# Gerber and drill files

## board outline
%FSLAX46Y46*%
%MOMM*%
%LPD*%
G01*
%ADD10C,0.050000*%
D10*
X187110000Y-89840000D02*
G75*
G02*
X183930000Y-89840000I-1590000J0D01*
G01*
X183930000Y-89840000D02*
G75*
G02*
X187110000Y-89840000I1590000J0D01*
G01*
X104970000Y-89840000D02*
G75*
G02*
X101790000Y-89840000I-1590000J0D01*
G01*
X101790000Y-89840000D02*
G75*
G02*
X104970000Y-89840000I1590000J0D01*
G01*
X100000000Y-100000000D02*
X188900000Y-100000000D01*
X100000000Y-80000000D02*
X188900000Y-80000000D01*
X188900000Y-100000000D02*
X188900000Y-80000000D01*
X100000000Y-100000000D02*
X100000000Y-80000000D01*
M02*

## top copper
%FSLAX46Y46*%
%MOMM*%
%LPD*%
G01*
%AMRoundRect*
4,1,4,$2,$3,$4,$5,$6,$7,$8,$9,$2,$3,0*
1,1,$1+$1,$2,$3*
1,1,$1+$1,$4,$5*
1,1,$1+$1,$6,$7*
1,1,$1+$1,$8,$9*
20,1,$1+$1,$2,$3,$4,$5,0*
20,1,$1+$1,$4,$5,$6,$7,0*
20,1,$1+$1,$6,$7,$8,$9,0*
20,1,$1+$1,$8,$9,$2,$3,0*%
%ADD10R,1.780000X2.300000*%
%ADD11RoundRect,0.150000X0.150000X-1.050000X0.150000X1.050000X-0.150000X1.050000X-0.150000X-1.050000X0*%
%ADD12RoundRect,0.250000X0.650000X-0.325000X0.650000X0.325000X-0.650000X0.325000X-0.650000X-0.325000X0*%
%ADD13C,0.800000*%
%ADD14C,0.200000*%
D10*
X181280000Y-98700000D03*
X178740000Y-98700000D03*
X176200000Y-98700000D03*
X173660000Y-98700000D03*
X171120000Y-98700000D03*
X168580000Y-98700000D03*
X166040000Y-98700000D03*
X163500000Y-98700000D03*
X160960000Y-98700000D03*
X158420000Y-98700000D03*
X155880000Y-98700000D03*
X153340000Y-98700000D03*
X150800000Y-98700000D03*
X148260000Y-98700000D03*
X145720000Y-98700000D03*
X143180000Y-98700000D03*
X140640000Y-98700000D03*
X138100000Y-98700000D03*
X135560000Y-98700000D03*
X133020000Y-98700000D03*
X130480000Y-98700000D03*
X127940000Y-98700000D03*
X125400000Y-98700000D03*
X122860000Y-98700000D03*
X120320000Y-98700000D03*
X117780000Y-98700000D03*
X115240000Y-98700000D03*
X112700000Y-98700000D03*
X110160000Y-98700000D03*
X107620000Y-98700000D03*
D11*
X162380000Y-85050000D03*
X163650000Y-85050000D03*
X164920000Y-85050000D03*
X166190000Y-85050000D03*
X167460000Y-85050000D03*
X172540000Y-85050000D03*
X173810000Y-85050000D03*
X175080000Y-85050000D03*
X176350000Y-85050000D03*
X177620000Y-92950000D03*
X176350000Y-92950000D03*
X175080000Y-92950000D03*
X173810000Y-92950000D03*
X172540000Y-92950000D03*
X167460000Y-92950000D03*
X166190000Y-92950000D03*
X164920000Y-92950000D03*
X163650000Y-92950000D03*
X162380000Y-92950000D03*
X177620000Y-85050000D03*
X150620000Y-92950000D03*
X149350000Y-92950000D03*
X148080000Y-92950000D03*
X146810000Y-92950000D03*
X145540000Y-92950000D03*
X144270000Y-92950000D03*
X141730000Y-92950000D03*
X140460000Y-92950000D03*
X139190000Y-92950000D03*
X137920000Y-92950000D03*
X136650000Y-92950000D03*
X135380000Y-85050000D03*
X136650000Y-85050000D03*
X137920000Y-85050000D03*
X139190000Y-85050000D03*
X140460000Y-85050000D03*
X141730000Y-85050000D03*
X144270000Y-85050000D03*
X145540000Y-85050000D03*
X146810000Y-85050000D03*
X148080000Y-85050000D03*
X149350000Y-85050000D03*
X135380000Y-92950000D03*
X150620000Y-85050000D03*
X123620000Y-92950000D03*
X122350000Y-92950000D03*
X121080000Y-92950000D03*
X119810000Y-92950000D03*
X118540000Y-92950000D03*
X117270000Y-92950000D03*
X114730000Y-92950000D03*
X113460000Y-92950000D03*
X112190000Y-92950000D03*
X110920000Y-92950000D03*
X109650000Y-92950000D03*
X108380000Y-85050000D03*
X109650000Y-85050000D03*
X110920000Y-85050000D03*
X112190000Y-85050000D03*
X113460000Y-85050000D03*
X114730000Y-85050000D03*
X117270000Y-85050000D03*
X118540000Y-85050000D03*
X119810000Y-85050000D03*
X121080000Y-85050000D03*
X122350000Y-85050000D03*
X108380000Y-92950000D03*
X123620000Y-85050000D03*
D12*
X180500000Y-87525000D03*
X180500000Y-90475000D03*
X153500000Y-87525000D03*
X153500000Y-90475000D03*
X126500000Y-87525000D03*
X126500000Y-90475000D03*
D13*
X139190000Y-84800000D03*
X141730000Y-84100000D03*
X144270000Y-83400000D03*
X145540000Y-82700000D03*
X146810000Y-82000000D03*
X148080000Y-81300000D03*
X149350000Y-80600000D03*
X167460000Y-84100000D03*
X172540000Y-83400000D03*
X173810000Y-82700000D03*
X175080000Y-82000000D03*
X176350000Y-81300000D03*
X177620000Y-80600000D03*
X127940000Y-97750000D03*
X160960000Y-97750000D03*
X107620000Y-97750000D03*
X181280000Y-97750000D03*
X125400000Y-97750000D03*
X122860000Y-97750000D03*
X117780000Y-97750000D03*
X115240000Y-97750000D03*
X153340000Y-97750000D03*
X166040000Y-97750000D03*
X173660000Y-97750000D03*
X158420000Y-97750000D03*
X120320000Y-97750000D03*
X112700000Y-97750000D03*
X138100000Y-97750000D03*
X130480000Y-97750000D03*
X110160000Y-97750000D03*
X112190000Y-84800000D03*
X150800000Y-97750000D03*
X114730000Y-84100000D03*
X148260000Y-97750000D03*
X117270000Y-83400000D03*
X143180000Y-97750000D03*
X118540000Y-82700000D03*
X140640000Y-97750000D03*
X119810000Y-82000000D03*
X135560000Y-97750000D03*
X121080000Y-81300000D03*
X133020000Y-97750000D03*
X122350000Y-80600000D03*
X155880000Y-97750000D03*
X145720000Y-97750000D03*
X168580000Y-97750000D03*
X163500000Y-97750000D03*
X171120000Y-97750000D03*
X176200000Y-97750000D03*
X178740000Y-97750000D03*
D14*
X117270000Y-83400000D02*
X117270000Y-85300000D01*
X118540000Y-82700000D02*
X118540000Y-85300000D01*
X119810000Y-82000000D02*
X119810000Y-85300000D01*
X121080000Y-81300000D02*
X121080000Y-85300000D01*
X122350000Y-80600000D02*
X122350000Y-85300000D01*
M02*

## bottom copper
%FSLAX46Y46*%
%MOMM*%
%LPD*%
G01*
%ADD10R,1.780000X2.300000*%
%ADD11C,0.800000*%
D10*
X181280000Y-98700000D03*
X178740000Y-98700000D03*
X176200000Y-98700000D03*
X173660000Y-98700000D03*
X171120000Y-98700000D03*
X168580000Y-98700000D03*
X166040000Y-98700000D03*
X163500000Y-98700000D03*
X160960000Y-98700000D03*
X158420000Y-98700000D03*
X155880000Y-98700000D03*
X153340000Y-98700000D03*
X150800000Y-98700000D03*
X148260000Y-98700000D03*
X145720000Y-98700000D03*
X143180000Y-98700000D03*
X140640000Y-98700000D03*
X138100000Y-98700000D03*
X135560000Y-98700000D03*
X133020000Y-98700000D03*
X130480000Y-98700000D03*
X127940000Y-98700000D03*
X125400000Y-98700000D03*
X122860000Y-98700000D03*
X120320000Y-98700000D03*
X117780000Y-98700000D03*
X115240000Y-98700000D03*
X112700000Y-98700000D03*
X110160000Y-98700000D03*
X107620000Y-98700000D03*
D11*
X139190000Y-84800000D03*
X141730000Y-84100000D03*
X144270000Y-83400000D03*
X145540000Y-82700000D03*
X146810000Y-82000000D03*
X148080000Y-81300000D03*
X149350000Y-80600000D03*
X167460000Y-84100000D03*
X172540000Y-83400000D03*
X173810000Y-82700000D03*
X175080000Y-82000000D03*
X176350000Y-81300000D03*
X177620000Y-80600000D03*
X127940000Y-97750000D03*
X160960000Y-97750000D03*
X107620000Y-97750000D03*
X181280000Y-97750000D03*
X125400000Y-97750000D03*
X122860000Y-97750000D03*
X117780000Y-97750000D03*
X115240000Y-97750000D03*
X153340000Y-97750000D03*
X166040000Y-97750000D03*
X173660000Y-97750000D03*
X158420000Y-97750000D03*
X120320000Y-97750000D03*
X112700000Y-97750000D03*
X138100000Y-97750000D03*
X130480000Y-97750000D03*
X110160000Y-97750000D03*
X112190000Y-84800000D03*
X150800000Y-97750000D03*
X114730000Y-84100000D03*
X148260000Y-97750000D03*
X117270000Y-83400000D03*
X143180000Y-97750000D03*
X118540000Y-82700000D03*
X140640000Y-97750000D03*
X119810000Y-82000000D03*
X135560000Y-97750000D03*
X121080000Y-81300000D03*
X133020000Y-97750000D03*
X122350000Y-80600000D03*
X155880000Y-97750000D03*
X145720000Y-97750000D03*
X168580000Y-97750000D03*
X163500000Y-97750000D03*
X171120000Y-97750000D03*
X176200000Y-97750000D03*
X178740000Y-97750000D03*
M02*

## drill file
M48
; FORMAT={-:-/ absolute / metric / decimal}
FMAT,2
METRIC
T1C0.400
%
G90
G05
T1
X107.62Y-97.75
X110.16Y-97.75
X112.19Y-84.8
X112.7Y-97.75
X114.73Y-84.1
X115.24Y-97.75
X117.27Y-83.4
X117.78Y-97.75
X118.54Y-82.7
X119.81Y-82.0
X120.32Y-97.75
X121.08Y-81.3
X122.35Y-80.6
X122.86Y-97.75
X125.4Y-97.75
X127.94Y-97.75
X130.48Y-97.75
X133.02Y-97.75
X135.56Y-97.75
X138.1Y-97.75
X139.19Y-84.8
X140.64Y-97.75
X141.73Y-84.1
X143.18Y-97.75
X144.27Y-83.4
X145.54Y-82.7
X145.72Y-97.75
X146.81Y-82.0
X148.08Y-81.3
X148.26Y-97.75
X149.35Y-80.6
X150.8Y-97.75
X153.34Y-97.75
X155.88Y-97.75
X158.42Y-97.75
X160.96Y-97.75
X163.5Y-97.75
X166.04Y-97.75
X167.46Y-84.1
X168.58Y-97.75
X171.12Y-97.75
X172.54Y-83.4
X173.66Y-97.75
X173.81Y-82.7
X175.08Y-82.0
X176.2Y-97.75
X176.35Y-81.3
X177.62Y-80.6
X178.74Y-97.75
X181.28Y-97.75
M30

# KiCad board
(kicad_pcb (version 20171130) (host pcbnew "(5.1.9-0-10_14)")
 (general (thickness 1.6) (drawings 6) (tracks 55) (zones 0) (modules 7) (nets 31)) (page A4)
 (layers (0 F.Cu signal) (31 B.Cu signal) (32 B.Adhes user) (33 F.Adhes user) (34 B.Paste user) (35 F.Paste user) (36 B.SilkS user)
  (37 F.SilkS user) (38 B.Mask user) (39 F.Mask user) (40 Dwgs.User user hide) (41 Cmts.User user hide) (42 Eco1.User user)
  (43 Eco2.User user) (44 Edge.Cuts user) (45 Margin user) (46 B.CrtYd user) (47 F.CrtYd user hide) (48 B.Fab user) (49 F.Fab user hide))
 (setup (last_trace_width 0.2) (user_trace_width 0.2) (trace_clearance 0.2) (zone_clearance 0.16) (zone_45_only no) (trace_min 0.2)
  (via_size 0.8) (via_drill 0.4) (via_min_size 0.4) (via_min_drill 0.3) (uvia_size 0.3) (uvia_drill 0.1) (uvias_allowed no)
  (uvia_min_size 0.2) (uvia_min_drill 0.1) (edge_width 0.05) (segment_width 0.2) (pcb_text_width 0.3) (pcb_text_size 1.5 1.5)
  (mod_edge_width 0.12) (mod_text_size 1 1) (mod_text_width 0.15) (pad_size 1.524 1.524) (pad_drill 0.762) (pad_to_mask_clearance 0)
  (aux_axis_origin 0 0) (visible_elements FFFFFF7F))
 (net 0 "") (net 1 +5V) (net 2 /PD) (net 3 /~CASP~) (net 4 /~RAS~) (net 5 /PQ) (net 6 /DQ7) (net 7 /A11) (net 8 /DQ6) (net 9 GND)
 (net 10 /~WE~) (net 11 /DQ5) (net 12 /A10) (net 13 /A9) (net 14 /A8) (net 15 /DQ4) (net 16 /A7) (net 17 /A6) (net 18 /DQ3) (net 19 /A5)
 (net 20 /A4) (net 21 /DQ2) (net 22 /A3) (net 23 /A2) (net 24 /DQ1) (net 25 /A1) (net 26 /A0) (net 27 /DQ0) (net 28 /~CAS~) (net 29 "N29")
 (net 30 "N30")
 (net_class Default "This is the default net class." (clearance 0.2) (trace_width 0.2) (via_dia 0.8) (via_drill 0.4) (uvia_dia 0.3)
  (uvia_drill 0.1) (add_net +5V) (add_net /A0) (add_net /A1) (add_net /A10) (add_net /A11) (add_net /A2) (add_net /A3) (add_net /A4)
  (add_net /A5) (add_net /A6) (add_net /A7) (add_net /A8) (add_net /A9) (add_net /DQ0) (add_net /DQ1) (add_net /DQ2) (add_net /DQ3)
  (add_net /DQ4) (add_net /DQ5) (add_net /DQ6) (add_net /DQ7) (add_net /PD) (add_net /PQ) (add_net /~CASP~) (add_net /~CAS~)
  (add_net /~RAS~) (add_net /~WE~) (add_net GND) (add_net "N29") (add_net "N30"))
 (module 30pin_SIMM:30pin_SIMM (layer F.Cu) (at 100 100)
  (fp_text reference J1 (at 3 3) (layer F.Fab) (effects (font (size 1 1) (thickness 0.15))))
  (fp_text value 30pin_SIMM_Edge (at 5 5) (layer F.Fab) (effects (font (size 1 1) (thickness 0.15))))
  (pad 30 connect rect (at 81.28 -1.3) (size 1.78 2.3) (layers B.Cu B.Mask) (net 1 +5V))
  (pad 29 connect rect (at 78.74 -1.3) (size 1.78 2.3) (layers B.Cu B.Mask) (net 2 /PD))
  (pad 28 connect rect (at 76.2 -1.3) (size 1.78 2.3) (layers B.Cu B.Mask) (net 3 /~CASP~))
  (pad 27 connect rect (at 73.66 -1.3) (size 1.78 2.3) (layers B.Cu B.Mask) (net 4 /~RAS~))
  (pad 26 connect rect (at 71.12 -1.3) (size 1.78 2.3) (layers B.Cu B.Mask) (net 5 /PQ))
  (pad 25 connect rect (at 68.58 -1.3) (size 1.78 2.3) (layers B.Cu B.Mask) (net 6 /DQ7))
  (pad 24 connect rect (at 66.04 -1.3) (size 1.78 2.3) (layers B.Cu B.Mask) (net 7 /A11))
  (pad 23 connect rect (at 63.5 -1.3) (size 1.78 2.3) (layers B.Cu B.Mask) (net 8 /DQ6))
  (pad 22 connect rect (at 60.96 -1.3) (size 1.78 2.3) (layers B.Cu B.Mask) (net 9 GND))
  (pad 21 connect rect (at 58.42 -1.3) (size 1.78 2.3) (layers B.Cu B.Mask) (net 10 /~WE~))
  (pad 20 connect rect (at 55.88 -1.3) (size 1.78 2.3) (layers B.Cu B.Mask) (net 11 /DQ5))
  (pad 19 connect rect (at 53.34 -1.3) (size 1.78 2.3) (layers B.Cu B.Mask) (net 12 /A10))
  (pad 18 connect rect (at 50.8 -1.3) (size 1.78 2.3) (layers B.Cu B.Mask) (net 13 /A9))
  (pad 17 connect rect (at 48.26 -1.3) (size 1.78 2.3) (layers B.Cu B.Mask) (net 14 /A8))
  (pad 16 connect rect (at 45.72 -1.3) (size 1.78 2.3) (layers B.Cu B.Mask) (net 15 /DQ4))
  (pad 15 connect rect (at 43.18 -1.3) (size 1.78 2.3) (layers B.Cu B.Mask) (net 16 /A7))
  (pad 14 connect rect (at 40.64 -1.3) (size 1.78 2.3) (layers B.Cu B.Mask) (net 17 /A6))
  (pad 13 connect rect (at 38.1 -1.3) (size 1.78 2.3) (layers B.Cu B.Mask) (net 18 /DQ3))
  (pad 12 connect rect (at 35.56 -1.3) (size 1.78 2.3) (layers B.Cu B.Mask) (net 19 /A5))
  (pad 11 connect rect (at 33.02 -1.3) (size 1.78 2.3) (layers B.Cu B.Mask) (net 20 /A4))
  (pad 10 connect rect (at 30.48 -1.3) (size 1.78 2.3) (layers B.Cu B.Mask) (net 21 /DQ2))
  (pad 9 connect rect (at 27.94 -1.3) (size 1.78 2.3) (layers B.Cu B.Mask) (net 9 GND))
  (pad 8 connect rect (at 25.4 -1.3) (size 1.78 2.3) (layers B.Cu B.Mask) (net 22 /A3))
  (pad 7 connect rect (at 22.86 -1.3) (size 1.78 2.3) (layers B.Cu B.Mask) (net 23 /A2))
  (pad 6 connect rect (at 20.32 -1.3) (size 1.78 2.3) (layers B.Cu B.Mask) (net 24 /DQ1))
  (pad 5 connect rect (at 17.78 -1.3) (size 1.78 2.3) (layers B.Cu B.Mask) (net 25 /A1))
  (pad 4 connect rect (at 15.24 -1.3) (size 1.78 2.3) (layers B.Cu B.Mask) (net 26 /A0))
  (pad 3 connect rect (at 12.7 -1.3) (size 1.78 2.3) (layers B.Cu B.Mask) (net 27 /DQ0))
  (pad 2 connect rect (at 10.16 -1.3) (size 1.78 2.3) (layers B.Cu B.Mask) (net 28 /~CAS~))
  (pad 30 connect rect (at 81.28 -1.3) (size 1.78 2.3) (layers F.Cu F.Mask) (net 1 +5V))
  (pad 29 connect rect (at 78.74 -1.3) (size 1.78 2.3) (layers F.Cu F.Mask) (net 2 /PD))
  (pad 28 connect rect (at 76.2 -1.3) (size 1.78 2.3) (layers F.Cu F.Mask) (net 3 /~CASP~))
  (pad 27 connect rect (at 73.66 -1.3) (size 1.78 2.3) (layers F.Cu F.Mask) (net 4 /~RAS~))
  (pad 26 connect rect (at 71.12 -1.3) (size 1.78 2.3) (layers F.Cu F.Mask) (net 5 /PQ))
  (pad 25 connect rect (at 68.58 -1.3) (size 1.78 2.3) (layers F.Cu F.Mask) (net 6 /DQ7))
  (pad 24 connect rect (at 66.04 -1.3) (size 1.78 2.3) (layers F.Cu F.Mask) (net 7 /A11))
  (pad 23 connect rect (at 63.5 -1.3) (size 1.78 2.3) (layers F.Cu F.Mask) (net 8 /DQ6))
  (pad 22 connect rect (at 60.96 -1.3) (size 1.78 2.3) (layers F.Cu F.Mask) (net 9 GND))
  (pad 21 connect rect (at 58.42 -1.3) (size 1.78 2.3) (layers F.Cu F.Mask) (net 10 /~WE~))
  (pad 20 connect rect (at 55.88 -1.3) (size 1.78 2.3) (layers F.Cu F.Mask) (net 11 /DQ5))
  (pad 19 connect rect (at 53.34 -1.3) (size 1.78 2.3) (layers F.Cu F.Mask) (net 12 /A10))
  (pad 18 connect rect (at 50.8 -1.3) (size 1.78 2.3) (layers F.Cu F.Mask) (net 13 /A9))
  (pad 17 connect rect (at 48.26 -1.3) (size 1.78 2.3) (layers F.Cu F.Mask) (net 14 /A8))
  (pad 16 connect rect (at 45.72 -1.3) (size 1.78 2.3) (layers F.Cu F.Mask) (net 15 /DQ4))
  (pad 15 connect rect (at 43.18 -1.3) (size 1.78 2.3) (layers F.Cu F.Mask) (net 16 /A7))
  (pad 14 connect rect (at 40.64 -1.3) (size 1.78 2.3) (layers F.Cu F.Mask) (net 17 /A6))
  (pad 13 connect rect (at 38.1 -1.3) (size 1.78 2.3) (layers F.Cu F.Mask) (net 18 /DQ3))
  (pad 12 connect rect (at 35.56 -1.3) (size 1.78 2.3) (layers F.Cu F.Mask) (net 19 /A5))
  (pad 11 connect rect (at 33.02 -1.3) (size 1.78 2.3) (layers F.Cu F.Mask) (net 20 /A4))
  (pad 10 connect rect (at 30.48 -1.3) (size 1.78 2.3) (layers F.Cu F.Mask) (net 21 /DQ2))
  (pad 9 connect rect (at 27.94 -1.3) (size 1.78 2.3) (layers F.Cu F.Mask) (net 9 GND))
  (pad 8 connect rect (at 25.4 -1.3) (size 1.78 2.3) (layers F.Cu F.Mask) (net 22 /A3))
  (pad 7 connect rect (at 22.86 -1.3) (size 1.78 2.3) (layers F.Cu F.Mask) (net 23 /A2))
  (pad 6 connect rect (at 20.32 -1.3) (size 1.78 2.3) (layers F.Cu F.Mask) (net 24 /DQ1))
  (pad 5 connect rect (at 17.78 -1.3) (size 1.78 2.3) (layers F.Cu F.Mask) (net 25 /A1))
  (pad 4 connect rect (at 15.24 -1.3) (size 1.78 2.3) (layers F.Cu F.Mask) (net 26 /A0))
  (pad 3 connect rect (at 12.7 -1.3) (size 1.78 2.3) (layers F.Cu F.Mask) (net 27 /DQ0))
  (pad 2 connect rect (at 10.16 -1.3) (size 1.78 2.3) (layers F.Cu F.Mask) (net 28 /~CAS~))
  (pad 1 connect rect (at 7.62 -1.3) (size 1.78 2.3) (layers F.Cu F.Mask) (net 1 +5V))
  (pad 1 connect rect (at 7.62 -1.3) (size 1.78 2.3) (layers B.Cu B.Mask) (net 1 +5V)))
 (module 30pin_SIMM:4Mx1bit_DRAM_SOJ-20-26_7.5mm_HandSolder (layer F.Cu) (at 170 89 90)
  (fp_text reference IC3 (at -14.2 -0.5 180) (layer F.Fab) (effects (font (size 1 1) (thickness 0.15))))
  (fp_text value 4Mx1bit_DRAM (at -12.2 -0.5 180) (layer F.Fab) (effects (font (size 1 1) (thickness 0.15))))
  (pad 26 smd roundrect (at 3.7 -7.62 90) (size 2.4 0.6) (drill (offset 0.25 0)) (layers F.Cu F.Paste F.Mask) (roundrect_rratio 0.25)
   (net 9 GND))
  (pad 25 smd roundrect (at 3.7 -6.35 90) (size 2.4 0.6) (drill (offset 0.25 0)) (layers F.Cu F.Paste F.Mask) (roundrect_rratio 0.25)
   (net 5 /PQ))
  (pad 24 smd roundrect (at 3.7 -5.08 90) (size 2.4 0.6) (drill (offset 0.25 0)) (layers F.Cu F.Paste F.Mask) (roundrect_rratio 0.25)
   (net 3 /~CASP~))
  (pad 23 smd roundrect (at 3.7 -3.81 90) (size 2.4 0.6) (drill (offset 0.25 0)) (layers F.Cu F.Paste F.Mask) (roundrect_rratio 0.25)
   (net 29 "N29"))
  (pad 22 smd roundrect (at 3.7 -2.54 90) (size 2.4 0.6) (drill (offset 0.25 0)) (layers F.Cu F.Paste F.Mask) (roundrect_rratio 0.25)
   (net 13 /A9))
  (pad 18 smd roundrect (at 3.7 2.54 90) (size 2.4 0.6) (drill (offset 0.25 0)) (layers F.Cu F.Paste F.Mask) (roundrect_rratio 0.25)
   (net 14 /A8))
  (pad 17 smd roundrect (at 3.7 3.81 90) (size 2.4 0.6) (drill (offset 0.25 0)) (layers F.Cu F.Paste F.Mask) (roundrect_rratio 0.25)
   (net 16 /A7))
  (pad 16 smd roundrect (at 3.7 5.08 90) (size 2.4 0.6) (drill (offset 0.25 0)) (layers F.Cu F.Paste F.Mask) (roundrect_rratio 0.25)
   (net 17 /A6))
  (pad 15 smd roundrect (at 3.7 6.35 90) (size 2.4 0.6) (drill (offset 0.25 0)) (layers F.Cu F.Paste F.Mask) (roundrect_rratio 0.25)
   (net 19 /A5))
  (pad 13 smd roundrect (at -3.7 7.62 90) (size 2.4 0.6) (drill (offset -0.25 0)) (layers F.Cu F.Paste F.Mask) (roundrect_rratio 0.25)
   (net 1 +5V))
  (pad 12 smd roundrect (at -3.7 6.35 90) (size 2.4 0.6) (drill (offset -0.25 0)) (layers F.Cu F.Paste F.Mask) (roundrect_rratio 0.25)
   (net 22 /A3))
  (pad 11 smd roundrect (at -3.7 5.08 90) (size 2.4 0.6) (drill (offset -0.25 0)) (layers F.Cu F.Paste F.Mask) (roundrect_rratio 0.25)
   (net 23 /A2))
  (pad 10 smd roundrect (at -3.7 3.81 90) (size 2.4 0.6) (drill (offset -0.25 0)) (layers F.Cu F.Paste F.Mask) (roundrect_rratio 0.25)
   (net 25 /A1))
  (pad 9 smd roundrect (at -3.7 2.54 90) (size 2.4 0.6) (drill (offset -0.25 0)) (layers F.Cu F.Paste F.Mask) (roundrect_rratio 0.25)
   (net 26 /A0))
  (pad 5 smd roundrect (at -3.7 -2.54 90) (size 2.4 0.6) (drill (offset -0.25 0)) (layers F.Cu F.Paste F.Mask) (roundrect_rratio 0.25)
   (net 12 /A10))
  (pad 4 smd roundrect (at -3.7 -3.81 90) (size 2.4 0.6) (drill (offset -0.25 0)) (layers F.Cu F.Paste F.Mask) (roundrect_rratio 0.25)
   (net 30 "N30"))
  (pad 3 smd roundrect (at -3.7 -5.08 90) (size 2.4 0.6) (drill (offset -0.25 0)) (layers F.Cu F.Paste F.Mask) (roundrect_rratio 0.25)
   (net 4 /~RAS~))
  (pad 2 smd roundrect (at -3.7 -6.35 90) (size 2.4 0.6) (drill (offset -0.25 0)) (layers F.Cu F.Paste F.Mask) (roundrect_rratio 0.25)
   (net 10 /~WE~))
  (pad 1 smd roundrect (at -3.7 -7.62 90) (size 2.4 0.6) (drill (offset -0.25 0)) (layers F.Cu F.Paste F.Mask) (roundrect_rratio 0.25)
   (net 2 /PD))
  (pad 14 smd roundrect (at 3.7 7.62 90) (size 2.4 0.6) (drill (offset 0.25 0)) (layers F.Cu F.Paste F.Mask) (roundrect_rratio 0.25)
   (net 20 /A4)))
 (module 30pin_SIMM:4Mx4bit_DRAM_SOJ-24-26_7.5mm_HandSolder (layer F.Cu) (at 143 89 90)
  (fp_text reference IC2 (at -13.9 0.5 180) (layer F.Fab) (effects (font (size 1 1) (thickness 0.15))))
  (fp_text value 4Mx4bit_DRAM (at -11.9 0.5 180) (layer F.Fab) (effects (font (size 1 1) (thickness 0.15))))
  (pad 13 smd roundrect (at -3.7 7.62 90) (size 2.4 0.6) (drill (offset -0.25 0)) (layers F.Cu F.Paste F.Mask) (roundrect_rratio 0.25)
   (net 1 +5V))
  (pad 12 smd roundrect (at -3.7 6.35 90) (size 2.4 0.6) (drill (offset -0.25 0)) (layers F.Cu F.Paste F.Mask) (roundrect_rratio 0.25)
   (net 22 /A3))
  (pad 11 smd roundrect (at -3.7 5.08 90) (size 2.4 0.6) (drill (offset -0.25 0)) (layers F.Cu F.Paste F.Mask) (roundrect_rratio 0.25)
   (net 23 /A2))
  (pad 10 smd roundrect (at -3.7 3.81 90) (size 2.4 0.6) (drill (offset -0.25 0)) (layers F.Cu F.Paste F.Mask) (roundrect_rratio 0.25)
   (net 25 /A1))
  (pad 9 smd roundrect (at -3.7 2.54 90) (size 2.4 0.6) (drill (offset -0.25 0)) (layers F.Cu F.Paste F.Mask) (roundrect_rratio 0.25)
   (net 26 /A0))
  (pad 8 smd roundrect (at -3.7 1.27 90) (size 2.4 0.6) (drill (offset -0.25 0)) (layers F.Cu F.Paste F.Mask) (roundrect_rratio 0.25)
   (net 12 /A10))
  (pad 6 smd roundrect (at -3.7 -1.27 90) (size 2.4 0.6) (drill (offset -0.25 0)) (layers F.Cu F.Paste F.Mask) (roundrect_rratio 0.25)
   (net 7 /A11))
  (pad 5 smd roundrect (at -3.7 -2.54 90) (size 2.4 0.6) (drill (offset -0.25 0)) (layers F.Cu F.Paste F.Mask) (roundrect_rratio 0.25)
   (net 4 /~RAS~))
  (pad 4 smd roundrect (at -3.7 -3.81 90) (size 2.4 0.6) (drill (offset -0.25 0)) (layers F.Cu F.Paste F.Mask) (roundrect_rratio 0.25)
   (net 10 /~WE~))
  (pad 3 smd roundrect (at -3.7 -5.08 90) (size 2.4 0.6) (drill (offset -0.25 0)) (layers F.Cu F.Paste F.Mask) (roundrect_rratio 0.25)
   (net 11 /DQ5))
  (pad 2 smd roundrect (at -3.7 -6.35 90) (size 2.4 0.6) (drill (offset -0.25 0)) (layers F.Cu F.Paste F.Mask) (roundrect_rratio 0.25)
   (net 15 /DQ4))
  (pad 26 smd roundrect (at 3.7 -7.62 90) (size 2.4 0.6) (drill (offset 0.25 0)) (layers F.Cu F.Paste F.Mask) (roundrect_rratio 0.25)
   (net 9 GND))
  (pad 25 smd roundrect (at 3.7 -6.35 90) (size 2.4 0.6) (drill (offset 0.25 0)) (layers F.Cu F.Paste F.Mask) (roundrect_rratio 0.25)
   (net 6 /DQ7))
  (pad 24 smd roundrect (at 3.7 -5.08 90) (size 2.4 0.6) (drill (offset 0.25 0)) (layers F.Cu F.Paste F.Mask) (roundrect_rratio 0.25)
   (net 8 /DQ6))
  (pad 23 smd roundrect (at 3.7 -3.81 90) (size 2.4 0.6) (drill (offset 0.25 0)) (layers F.Cu F.Paste F.Mask) (roundrect_rratio 0.25)
   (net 28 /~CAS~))
  (pad 22 smd roundrect (at 3.7 -2.54 90) (size 2.4 0.6) (drill (offset 0.25 0)) (layers F.Cu F.Paste F.Mask) (roundrect_rratio 0.25)
   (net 9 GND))
  (pad 21 smd roundrect (at 3.7 -1.27 90) (size 2.4 0.6) (drill (offset 0.25 0)) (layers F.Cu F.Paste F.Mask) (roundrect_rratio 0.25)
   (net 13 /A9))
  (pad 19 smd roundrect (at 3.7 1.27 90) (size 2.4 0.6) (drill (offset 0.25 0)) (layers F.Cu F.Paste F.Mask) (roundrect_rratio 0.25)
   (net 14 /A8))
  (pad 18 smd roundrect (at 3.7 2.54 90) (size 2.4 0.6) (drill (offset 0.25 0)) (layers F.Cu F.Paste F.Mask) (roundrect_rratio 0.25)
   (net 16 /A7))
  (pad 17 smd roundrect (at 3.7 3.81 90) (size 2.4 0.6) (drill (offset 0.25 0)) (layers F.Cu F.Paste F.Mask) (roundrect_rratio 0.25)
   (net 17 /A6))
  (pad 16 smd roundrect (at 3.7 5.08 90) (size 2.4 0.6) (drill (offset 0.25 0)) (layers F.Cu F.Paste F.Mask) (roundrect_rratio 0.25)
   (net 19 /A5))
  (pad 15 smd roundrect (at 3.7 6.35 90) (size 2.4 0.6) (drill (offset 0.25 0)) (layers F.Cu F.Paste F.Mask) (roundrect_rratio 0.25)
   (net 20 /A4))
  (pad 1 smd roundrect (at -3.7 -7.62 90) (size 2.4 0.6) (drill (offset -0.25 0)) (layers F.Cu F.Paste F.Mask) (roundrect_rratio 0.25)
   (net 1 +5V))
  (pad 14 smd roundrect (at 3.7 7.62 90) (size 2.4 0.6) (drill (offset 0.25 0)) (layers F.Cu F.Paste F.Mask) (roundrect_rratio 0.25)
   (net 9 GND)))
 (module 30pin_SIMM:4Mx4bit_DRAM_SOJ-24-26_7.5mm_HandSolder (layer F.Cu) (at 116 89 90)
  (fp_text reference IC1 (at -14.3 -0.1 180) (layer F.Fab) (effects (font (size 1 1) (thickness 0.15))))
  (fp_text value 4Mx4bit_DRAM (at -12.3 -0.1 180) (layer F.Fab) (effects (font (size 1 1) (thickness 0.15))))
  (pad 13 smd roundrect (at -3.7 7.62 90) (size 2.4 0.6) (drill (offset -0.25 0)) (layers F.Cu F.Paste F.Mask) (roundrect_rratio 0.25)
   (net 1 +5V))
  (pad 12 smd roundrect (at -3.7 6.35 90) (size 2.4 0.6) (drill (offset -0.25 0)) (layers F.Cu F.Paste F.Mask) (roundrect_rratio 0.25)
   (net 22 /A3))
  (pad 11 smd roundrect (at -3.7 5.08 90) (size 2.4 0.6) (drill (offset -0.25 0)) (layers F.Cu F.Paste F.Mask) (roundrect_rratio 0.25)
   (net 23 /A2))
  (pad 10 smd roundrect (at -3.7 3.81 90) (size 2.4 0.6) (drill (offset -0.25 0)) (layers F.Cu F.Paste F.Mask) (roundrect_rratio 0.25)
   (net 25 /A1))
  (pad 9 smd roundrect (at -3.7 2.54 90) (size 2.4 0.6) (drill (offset -0.25 0)) (layers F.Cu F.Paste F.Mask) (roundrect_rratio 0.25)
   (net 26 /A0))
  (pad 8 smd roundrect (at -3.7 1.27 90) (size 2.4 0.6) (drill (offset -0.25 0)) (layers F.Cu F.Paste F.Mask) (roundrect_rratio 0.25)
   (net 12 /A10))
  (pad 6 smd roundrect (at -3.7 -1.27 90) (size 2.4 0.6) (drill (offset -0.25 0)) (layers F.Cu F.Paste F.Mask) (roundrect_rratio 0.25)
   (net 7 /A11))
  (pad 5 smd roundrect (at -3.7 -2.54 90) (size 2.4 0.6) (drill (offset -0.25 0)) (layers F.Cu F.Paste F.Mask) (roundrect_rratio 0.25)
   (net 4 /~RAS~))
  (pad 4 smd roundrect (at -3.7 -3.81 90) (size 2.4 0.6) (drill (offset -0.25 0)) (layers F.Cu F.Paste F.Mask) (roundrect_rratio 0.25)
   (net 10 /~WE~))
  (pad 3 smd roundrect (at -3.7 -5.08 90) (size 2.4 0.6) (drill (offset -0.25 0)) (layers F.Cu F.Paste F.Mask) (roundrect_rratio 0.25)
   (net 24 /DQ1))
  (pad 2 smd roundrect (at -3.7 -6.35 90) (size 2.4 0.6) (drill (offset -0.25 0)) (layers F.Cu F.Paste F.Mask) (roundrect_rratio 0.25)
   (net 27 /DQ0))
  (pad 26 smd roundrect (at 3.7 -7.62 90) (size 2.4 0.6) (drill (offset 0.25 0)) (layers F.Cu F.Paste F.Mask) (roundrect_rratio 0.25)
   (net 9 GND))
  (pad 25 smd roundrect (at 3.7 -6.35 90) (size 2.4 0.6) (drill (offset 0.25 0)) (layers F.Cu F.Paste F.Mask) (roundrect_rratio 0.25)
   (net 18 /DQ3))
  (pad 24 smd roundrect (at 3.7 -5.08 90) (size 2.4 0.6) (drill (offset 0.25 0)) (layers F.Cu F.Paste F.Mask) (roundrect_rratio 0.25)
   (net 21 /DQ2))
  (pad 23 smd roundrect (at 3.7 -3.81 90) (size 2.4 0.6) (drill (offset 0.25 0)) (layers F.Cu F.Paste F.Mask) (roundrect_rratio 0.25)
   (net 28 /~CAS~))
  (pad 22 smd roundrect (at 3.7 -2.54 90) (size 2.4 0.6) (drill (offset 0.25 0)) (layers F.Cu F.Paste F.Mask) (roundrect_rratio 0.25)
   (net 9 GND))
  (pad 21 smd roundrect (at 3.7 -1.27 90) (size 2.4 0.6) (drill (offset 0.25 0)) (layers F.Cu F.Paste F.Mask) (roundrect_rratio 0.25)
   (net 13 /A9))
  (pad 19 smd roundrect (at 3.7 1.27 90) (size 2.4 0.6) (drill (offset 0.25 0)) (layers F.Cu F.Paste F.Mask) (roundrect_rratio 0.25)
   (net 14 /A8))
  (pad 18 smd roundrect (at 3.7 2.54 90) (size 2.4 0.6) (drill (offset 0.25 0)) (layers F.Cu F.Paste F.Mask) (roundrect_rratio 0.25)
   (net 16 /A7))
  (pad 17 smd roundrect (at 3.7 3.81 90) (size 2.4 0.6) (drill (offset 0.25 0)) (layers F.Cu F.Paste F.Mask) (roundrect_rratio 0.25)
   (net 17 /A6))
  (pad 16 smd roundrect (at 3.7 5.08 90) (size 2.4 0.6) (drill (offset 0.25 0)) (layers F.Cu F.Paste F.Mask) (roundrect_rratio 0.25)
   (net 19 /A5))
  (pad 15 smd roundrect (at 3.7 6.35 90) (size 2.4 0.6) (drill (offset 0.25 0)) (layers F.Cu F.Paste F.Mask) (roundrect_rratio 0.25)
   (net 20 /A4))
  (pad 1 smd roundrect (at -3.7 -7.62 90) (size 2.4 0.6) (drill (offset -0.25 0)) (layers F.Cu F.Paste F.Mask) (roundrect_rratio 0.25)
   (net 1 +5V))
  (pad 14 smd roundrect (at 3.7 7.62 90) (size 2.4 0.6) (drill (offset 0.25 0)) (layers F.Cu F.Paste F.Mask) (roundrect_rratio 0.25)
   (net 9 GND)))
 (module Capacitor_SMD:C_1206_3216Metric (layer F.Cu) (at 180.5 89 90)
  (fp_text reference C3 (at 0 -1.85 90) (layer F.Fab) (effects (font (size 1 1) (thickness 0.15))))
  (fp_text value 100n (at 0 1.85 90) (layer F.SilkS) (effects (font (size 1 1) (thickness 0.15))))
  (pad 2 smd roundrect (at 1.475 0 90) (size 1.15 1.8) (layers F.Cu F.Paste F.Mask) (roundrect_rratio 0.217391) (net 9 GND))
  (pad 1 smd roundrect (at -1.475 0 90) (size 1.15 1.8) (layers F.Cu F.Paste F.Mask) (roundrect_rratio 0.217391) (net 1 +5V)))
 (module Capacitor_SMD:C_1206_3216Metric (layer F.Cu) (at 153.5 89 90)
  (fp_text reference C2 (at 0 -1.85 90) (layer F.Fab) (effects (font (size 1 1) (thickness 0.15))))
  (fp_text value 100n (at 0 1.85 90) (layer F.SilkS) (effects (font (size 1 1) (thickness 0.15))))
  (pad 2 smd roundrect (at 1.475 0 90) (size 1.15 1.8) (layers F.Cu F.Paste F.Mask) (roundrect_rratio 0.217391) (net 9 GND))
  (pad 1 smd roundrect (at -1.475 0 90) (size 1.15 1.8) (layers F.Cu F.Paste F.Mask) (roundrect_rratio 0.217391) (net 1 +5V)))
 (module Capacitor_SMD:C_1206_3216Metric (layer F.Cu) (at 126.5 89 90)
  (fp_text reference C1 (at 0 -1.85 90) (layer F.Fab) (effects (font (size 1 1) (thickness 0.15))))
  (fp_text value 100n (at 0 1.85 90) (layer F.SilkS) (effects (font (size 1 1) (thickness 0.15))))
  (pad 2 smd roundrect (at 1.475 0 90) (size 1.15 1.8) (layers F.Cu F.Paste F.Mask) (roundrect_rratio 0.217391) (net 9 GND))
  (pad 1 smd roundrect (at -1.475 0 90) (size 1.15 1.8) (layers F.Cu F.Paste F.Mask) (roundrect_rratio 0.217391) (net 1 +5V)))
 (gr_circle (center 185.52 89.84) (end 187.11 89.84) (layer Edge.Cuts) (width 0.05))
 (gr_circle (center 103.38 89.84) (end 104.97 89.84) (layer Edge.Cuts) (width 0.05))
 (gr_line (start 100 100) (end 188.9 100) (layer Edge.Cuts) (width 0.05))
 (gr_line (start 100 80) (end 188.9 80) (layer Edge.Cuts) (width 0.05))
 (gr_line (start 188.9 100) (end 188.9 80) (layer Edge.Cuts) (width 0.05))
 (gr_line (start 100 100) (end 100 80) (layer Edge.Cuts) (width 0.05))
 (via (at 139.19 84.8) (size 0.8) (drill 0.4) (layers F.Cu B.Cu) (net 28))
 (via (at 141.73 84.1) (size 0.8) (drill 0.4) (layers F.Cu B.Cu) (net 13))
 (via (at 144.27 83.4) (size 0.8) (drill 0.4) (layers F.Cu B.Cu) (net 14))
 (via (at 145.54 82.7) (size 0.8) (drill 0.4) (layers F.Cu B.Cu) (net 16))
 (via (at 146.81 82) (size 0.8) (drill 0.4) (layers F.Cu B.Cu) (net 17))
 (via (at 148.08 81.3) (size 0.8) (drill 0.4) (layers F.Cu B.Cu) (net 19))
 (via (at 149.35 80.6) (size 0.8) (drill 0.4) (layers F.Cu B.Cu) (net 20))
 (via (at 167.46 84.1) (size 0.8) (drill 0.4) (layers F.Cu B.Cu) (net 13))
 (via (at 172.54 83.4) (size 0.8) (drill 0.4) (layers F.Cu B.Cu) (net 14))
 (via (at 173.81 82.7) (size 0.8) (drill 0.4) (layers F.Cu B.Cu) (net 16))
 (via (at 175.08 82) (size 0.8) (drill 0.4) (layers F.Cu B.Cu) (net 17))
 (via (at 176.35 81.3) (size 0.8) (drill 0.4) (layers F.Cu B.Cu) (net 19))
 (via (at 177.62 80.6) (size 0.8) (drill 0.4) (layers F.Cu B.Cu) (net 20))
 (via (at 127.94 97.75) (size 0.8) (drill 0.4) (layers F.Cu B.Cu) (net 9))
 (via (at 160.96 97.75) (size 0.8) (drill 0.4) (layers F.Cu B.Cu) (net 9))
 (via (at 107.62 97.75) (size 0.8) (drill 0.4) (layers F.Cu B.Cu) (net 1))
 (via (at 181.28 97.75) (size 0.8) (drill 0.4) (layers F.Cu B.Cu) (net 1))
 (via (at 125.4 97.75) (size 0.8) (drill 0.4) (layers F.Cu B.Cu) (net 22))
 (via (at 122.86 97.75) (size 0.8) (drill 0.4) (layers F.Cu B.Cu) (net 23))
 (via (at 117.78 97.75) (size 0.8) (drill 0.4) (layers F.Cu B.Cu) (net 25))
 (via (at 115.24 97.75) (size 0.8) (drill 0.4) (layers F.Cu B.Cu) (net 26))
 (via (at 153.34 97.75) (size 0.8) (drill 0.4) (layers F.Cu B.Cu) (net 12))
 (via (at 166.04 97.75) (size 0.8) (drill 0.4) (layers F.Cu B.Cu) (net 7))
 (via (at 173.66 97.75) (size 0.8) (drill 0.4) (layers F.Cu B.Cu) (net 4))
 (via (at 158.42 97.75) (size 0.8) (drill 0.4) (layers F.Cu B.Cu) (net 10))
 (via (at 120.32 97.75) (size 0.8) (drill 0.4) (layers F.Cu B.Cu) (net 24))
 (via (at 112.7 97.75) (size 0.8) (drill 0.4) (layers F.Cu B.Cu) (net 27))
 (via (at 138.1 97.75) (size 0.8) (drill 0.4) (layers F.Cu B.Cu) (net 18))
 (via (at 130.48 97.75) (size 0.8) (drill 0.4) (layers F.Cu B.Cu) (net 21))
 (via (at 110.16 97.75) (size 0.8) (drill 0.4) (layers F.Cu B.Cu) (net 28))
 (via (at 112.19 84.8) (size 0.8) (drill 0.4) (layers F.Cu B.Cu) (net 28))
 (via (at 150.8 97.75) (size 0.8) (drill 0.4) (layers F.Cu B.Cu) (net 13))
 (via (at 114.73 84.1) (size 0.8) (drill 0.4) (layers F.Cu B.Cu) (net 13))
 (via (at 148.26 97.75) (size 0.8) (drill 0.4) (layers F.Cu B.Cu) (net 14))
 (via (at 117.27 83.4) (size 0.8) (drill 0.4) (layers F.Cu B.Cu) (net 14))
 (segment (start 117.27 83.4) (end 117.27 85.3) (width 0.2) (layer F.Cu) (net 14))
 (via (at 143.18 97.75) (size 0.8) (drill 0.4) (layers F.Cu B.Cu) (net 16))
 (via (at 118.54 82.7) (size 0.8) (drill 0.4) (layers F.Cu B.Cu) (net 16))
 (segment (start 118.54 82.7) (end 118.54 85.3) (width 0.2) (layer F.Cu) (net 16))
 (via (at 140.64 97.75) (size 0.8) (drill 0.4) (layers F.Cu B.Cu) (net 17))
 (via (at 119.81 82) (size 0.8) (drill 0.4) (layers F.Cu B.Cu) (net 17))
 (segment (start 119.81 82) (end 119.81 85.3) (width 0.2) (layer F.Cu) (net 17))
 (via (at 135.56 97.75) (size 0.8) (drill 0.4) (layers F.Cu B.Cu) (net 19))
 (via (at 121.08 81.3) (size 0.8) (drill 0.4) (layers F.Cu B.Cu) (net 19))
 (segment (start 121.08 81.3) (end 121.08 85.3) (width 0.2) (layer F.Cu) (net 19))
 (via (at 133.02 97.75) (size 0.8) (drill 0.4) (layers F.Cu B.Cu) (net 20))
 (via (at 122.35 80.6) (size 0.8) (drill 0.4) (layers F.Cu B.Cu) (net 20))
 (segment (start 122.35 80.6) (end 122.35 85.3) (width 0.2) (layer F.Cu) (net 20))
 (via (at 155.88 97.75) (size 0.8) (drill 0.4) (layers F.Cu B.Cu) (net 11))
 (via (at 145.72 97.75) (size 0.8) (drill 0.4) (layers F.Cu B.Cu) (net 15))
 (via (at 168.58 97.75) (size 0.8) (drill 0.4) (layers F.Cu B.Cu) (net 6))
 (via (at 163.5 97.75) (size 0.8) (drill 0.4) (layers F.Cu B.Cu) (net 8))
 (via (at 171.12 97.75) (size 0.8) (drill 0.4) (layers F.Cu B.Cu) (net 5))
 (via (at 176.2 97.75) (size 0.8) (drill 0.4) (layers F.Cu B.Cu) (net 3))
 (via (at 178.74 97.75) (size 0.8) (drill 0.4) (layers F.Cu B.Cu) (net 2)))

